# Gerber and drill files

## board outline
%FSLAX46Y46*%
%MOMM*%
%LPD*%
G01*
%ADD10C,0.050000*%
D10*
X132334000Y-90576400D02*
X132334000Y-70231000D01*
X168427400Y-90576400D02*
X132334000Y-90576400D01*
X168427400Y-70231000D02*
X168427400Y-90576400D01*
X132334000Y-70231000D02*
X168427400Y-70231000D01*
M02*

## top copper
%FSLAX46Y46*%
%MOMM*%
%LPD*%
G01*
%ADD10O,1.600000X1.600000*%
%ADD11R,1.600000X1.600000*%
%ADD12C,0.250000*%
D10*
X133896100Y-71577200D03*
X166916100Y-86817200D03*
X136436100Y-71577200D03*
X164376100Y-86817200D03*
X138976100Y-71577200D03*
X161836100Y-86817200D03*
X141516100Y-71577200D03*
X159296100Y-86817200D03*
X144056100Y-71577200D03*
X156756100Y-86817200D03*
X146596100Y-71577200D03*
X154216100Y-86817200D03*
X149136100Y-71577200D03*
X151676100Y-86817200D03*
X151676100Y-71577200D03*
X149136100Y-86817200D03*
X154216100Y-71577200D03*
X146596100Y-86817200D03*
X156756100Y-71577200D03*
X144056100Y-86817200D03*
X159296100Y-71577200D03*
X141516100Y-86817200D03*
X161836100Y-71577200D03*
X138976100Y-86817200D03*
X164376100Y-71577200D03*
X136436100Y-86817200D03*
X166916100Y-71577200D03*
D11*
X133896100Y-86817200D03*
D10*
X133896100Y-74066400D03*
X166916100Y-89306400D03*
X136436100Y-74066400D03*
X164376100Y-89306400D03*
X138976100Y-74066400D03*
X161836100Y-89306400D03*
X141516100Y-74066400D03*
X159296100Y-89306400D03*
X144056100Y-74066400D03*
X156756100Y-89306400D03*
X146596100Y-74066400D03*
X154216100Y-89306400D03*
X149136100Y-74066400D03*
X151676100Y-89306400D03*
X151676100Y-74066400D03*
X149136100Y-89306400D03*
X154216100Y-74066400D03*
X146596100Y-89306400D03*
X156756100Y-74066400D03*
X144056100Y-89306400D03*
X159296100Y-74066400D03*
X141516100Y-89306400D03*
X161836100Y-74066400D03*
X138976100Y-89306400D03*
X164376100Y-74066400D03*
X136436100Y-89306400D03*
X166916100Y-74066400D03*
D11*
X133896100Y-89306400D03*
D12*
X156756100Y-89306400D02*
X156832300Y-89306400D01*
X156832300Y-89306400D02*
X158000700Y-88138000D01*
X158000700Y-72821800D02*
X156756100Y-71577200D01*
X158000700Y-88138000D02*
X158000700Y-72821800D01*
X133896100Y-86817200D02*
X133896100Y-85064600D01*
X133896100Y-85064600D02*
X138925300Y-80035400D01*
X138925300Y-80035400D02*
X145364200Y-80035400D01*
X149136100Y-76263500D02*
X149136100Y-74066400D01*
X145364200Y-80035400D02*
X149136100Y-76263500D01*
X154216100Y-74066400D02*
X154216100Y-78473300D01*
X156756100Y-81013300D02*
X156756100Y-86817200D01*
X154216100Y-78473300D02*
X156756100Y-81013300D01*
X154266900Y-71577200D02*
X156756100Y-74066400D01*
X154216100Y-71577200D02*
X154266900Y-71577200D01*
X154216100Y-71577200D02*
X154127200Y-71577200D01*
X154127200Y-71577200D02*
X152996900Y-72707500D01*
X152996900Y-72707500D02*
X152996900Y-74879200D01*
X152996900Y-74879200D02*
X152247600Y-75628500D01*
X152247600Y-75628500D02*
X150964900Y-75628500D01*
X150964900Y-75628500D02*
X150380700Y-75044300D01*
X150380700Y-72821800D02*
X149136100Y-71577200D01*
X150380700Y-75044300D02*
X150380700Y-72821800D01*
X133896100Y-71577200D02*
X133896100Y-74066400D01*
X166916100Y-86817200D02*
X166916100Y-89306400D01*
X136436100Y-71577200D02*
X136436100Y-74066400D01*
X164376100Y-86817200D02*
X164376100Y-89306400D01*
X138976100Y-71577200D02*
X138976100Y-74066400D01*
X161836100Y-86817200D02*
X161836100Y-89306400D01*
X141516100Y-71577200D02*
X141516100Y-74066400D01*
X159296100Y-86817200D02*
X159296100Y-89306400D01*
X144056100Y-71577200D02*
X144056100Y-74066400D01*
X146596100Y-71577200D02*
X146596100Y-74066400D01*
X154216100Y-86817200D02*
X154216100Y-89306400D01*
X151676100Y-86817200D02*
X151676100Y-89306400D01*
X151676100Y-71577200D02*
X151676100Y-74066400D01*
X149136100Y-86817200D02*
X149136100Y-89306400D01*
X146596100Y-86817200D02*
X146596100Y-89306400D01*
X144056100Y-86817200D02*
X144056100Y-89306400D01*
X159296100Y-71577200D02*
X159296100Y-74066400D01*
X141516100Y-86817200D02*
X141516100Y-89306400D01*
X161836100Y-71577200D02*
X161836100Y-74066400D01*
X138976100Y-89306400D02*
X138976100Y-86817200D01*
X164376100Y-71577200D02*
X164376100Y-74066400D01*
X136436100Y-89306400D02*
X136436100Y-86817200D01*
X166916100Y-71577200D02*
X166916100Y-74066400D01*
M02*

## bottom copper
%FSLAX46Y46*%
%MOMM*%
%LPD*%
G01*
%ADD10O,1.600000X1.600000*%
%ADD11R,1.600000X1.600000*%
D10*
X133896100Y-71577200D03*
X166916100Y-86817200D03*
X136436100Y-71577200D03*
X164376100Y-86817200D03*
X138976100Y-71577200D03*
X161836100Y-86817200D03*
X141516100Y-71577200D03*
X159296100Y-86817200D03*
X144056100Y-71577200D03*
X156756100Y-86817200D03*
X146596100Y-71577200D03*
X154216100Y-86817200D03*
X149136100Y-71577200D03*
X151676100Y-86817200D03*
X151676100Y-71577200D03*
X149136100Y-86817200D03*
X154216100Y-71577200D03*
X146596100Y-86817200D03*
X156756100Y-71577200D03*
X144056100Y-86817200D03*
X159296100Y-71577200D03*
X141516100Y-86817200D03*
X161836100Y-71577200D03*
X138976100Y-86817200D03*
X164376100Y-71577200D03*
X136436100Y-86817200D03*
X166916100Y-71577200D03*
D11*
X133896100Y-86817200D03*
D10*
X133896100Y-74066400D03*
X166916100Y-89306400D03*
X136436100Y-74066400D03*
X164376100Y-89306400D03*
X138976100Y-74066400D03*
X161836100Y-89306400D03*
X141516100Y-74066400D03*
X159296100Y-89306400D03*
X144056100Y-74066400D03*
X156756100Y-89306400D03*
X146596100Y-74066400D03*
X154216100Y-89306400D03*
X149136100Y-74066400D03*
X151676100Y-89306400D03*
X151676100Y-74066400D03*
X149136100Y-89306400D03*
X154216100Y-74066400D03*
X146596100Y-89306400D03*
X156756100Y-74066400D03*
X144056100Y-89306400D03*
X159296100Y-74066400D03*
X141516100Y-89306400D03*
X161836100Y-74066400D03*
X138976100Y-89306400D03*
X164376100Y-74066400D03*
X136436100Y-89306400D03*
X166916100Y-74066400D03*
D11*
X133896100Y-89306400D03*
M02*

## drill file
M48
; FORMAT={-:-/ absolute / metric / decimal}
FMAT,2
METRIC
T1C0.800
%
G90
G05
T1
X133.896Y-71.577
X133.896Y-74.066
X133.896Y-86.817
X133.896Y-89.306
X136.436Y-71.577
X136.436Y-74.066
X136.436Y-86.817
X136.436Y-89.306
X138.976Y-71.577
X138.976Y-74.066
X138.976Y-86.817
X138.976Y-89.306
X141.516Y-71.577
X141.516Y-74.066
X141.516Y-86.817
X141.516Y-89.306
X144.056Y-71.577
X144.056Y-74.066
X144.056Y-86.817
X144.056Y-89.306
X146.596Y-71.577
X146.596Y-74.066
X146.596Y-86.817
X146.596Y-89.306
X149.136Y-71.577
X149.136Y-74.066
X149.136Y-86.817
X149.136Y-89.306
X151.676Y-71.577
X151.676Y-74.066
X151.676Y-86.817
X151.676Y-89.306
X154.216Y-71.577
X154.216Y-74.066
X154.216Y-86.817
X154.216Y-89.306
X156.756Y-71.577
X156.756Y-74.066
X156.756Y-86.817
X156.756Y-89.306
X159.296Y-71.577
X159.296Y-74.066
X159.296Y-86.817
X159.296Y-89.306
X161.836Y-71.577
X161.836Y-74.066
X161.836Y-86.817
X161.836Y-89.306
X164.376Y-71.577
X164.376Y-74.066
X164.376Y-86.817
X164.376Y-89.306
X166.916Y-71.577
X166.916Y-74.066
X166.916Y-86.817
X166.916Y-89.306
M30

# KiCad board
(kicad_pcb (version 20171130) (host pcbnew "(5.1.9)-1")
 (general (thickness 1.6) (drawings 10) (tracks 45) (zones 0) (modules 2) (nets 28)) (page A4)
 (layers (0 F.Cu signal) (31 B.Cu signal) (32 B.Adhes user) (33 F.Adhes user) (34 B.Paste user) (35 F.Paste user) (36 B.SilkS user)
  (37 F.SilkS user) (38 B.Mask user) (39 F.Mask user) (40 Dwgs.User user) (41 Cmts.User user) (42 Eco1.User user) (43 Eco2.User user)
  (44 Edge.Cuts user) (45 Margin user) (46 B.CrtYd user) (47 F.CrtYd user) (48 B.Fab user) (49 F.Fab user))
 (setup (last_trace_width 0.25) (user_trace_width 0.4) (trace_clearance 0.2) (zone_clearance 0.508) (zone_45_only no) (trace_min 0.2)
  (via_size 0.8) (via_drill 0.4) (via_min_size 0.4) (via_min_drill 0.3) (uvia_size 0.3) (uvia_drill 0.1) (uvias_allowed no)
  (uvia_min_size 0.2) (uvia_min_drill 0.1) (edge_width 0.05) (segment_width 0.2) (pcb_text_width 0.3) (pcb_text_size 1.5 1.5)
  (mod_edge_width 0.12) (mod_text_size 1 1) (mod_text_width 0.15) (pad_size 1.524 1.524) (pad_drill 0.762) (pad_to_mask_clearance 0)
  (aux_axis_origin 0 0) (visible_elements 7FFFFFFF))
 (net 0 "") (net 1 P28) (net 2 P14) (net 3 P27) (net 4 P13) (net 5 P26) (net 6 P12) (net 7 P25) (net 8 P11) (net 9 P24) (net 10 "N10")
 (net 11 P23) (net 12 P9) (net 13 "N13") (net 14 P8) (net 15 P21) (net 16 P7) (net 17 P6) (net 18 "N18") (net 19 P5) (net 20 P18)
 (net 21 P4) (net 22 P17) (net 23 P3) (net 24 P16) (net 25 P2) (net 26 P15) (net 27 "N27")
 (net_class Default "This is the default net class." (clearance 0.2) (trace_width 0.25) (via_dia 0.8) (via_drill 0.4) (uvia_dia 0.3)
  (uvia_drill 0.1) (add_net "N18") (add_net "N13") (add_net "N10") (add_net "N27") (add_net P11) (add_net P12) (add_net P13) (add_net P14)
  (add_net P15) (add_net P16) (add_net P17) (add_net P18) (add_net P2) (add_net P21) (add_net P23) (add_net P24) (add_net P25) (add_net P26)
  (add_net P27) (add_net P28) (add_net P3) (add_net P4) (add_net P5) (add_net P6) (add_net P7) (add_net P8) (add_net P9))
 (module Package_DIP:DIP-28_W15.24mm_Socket (layer F.Cu) (at 133.8961 86.8172 90)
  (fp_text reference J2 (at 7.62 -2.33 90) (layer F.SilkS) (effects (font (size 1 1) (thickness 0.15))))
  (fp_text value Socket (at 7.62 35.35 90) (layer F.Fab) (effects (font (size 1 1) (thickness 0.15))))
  (pad 28 thru_hole oval (at 15.24 0 90) (size 1.6 1.6) (drill 0.8) (layers *.Cu *.Mask) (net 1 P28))
  (pad 14 thru_hole oval (at 0 33.02 90) (size 1.6 1.6) (drill 0.8) (layers *.Cu *.Mask) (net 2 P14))
  (pad 27 thru_hole oval (at 15.24 2.54 90) (size 1.6 1.6) (drill 0.8) (layers *.Cu *.Mask) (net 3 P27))
  (pad 13 thru_hole oval (at 0 30.48 90) (size 1.6 1.6) (drill 0.8) (layers *.Cu *.Mask) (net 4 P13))
  (pad 26 thru_hole oval (at 15.24 5.08 90) (size 1.6 1.6) (drill 0.8) (layers *.Cu *.Mask) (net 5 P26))
  (pad 12 thru_hole oval (at 0 27.94 90) (size 1.6 1.6) (drill 0.8) (layers *.Cu *.Mask) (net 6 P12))
  (pad 25 thru_hole oval (at 15.24 7.62 90) (size 1.6 1.6) (drill 0.8) (layers *.Cu *.Mask) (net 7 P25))
  (pad 11 thru_hole oval (at 0 25.4 90) (size 1.6 1.6) (drill 0.8) (layers *.Cu *.Mask) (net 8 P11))
  (pad 24 thru_hole oval (at 15.24 10.16 90) (size 1.6 1.6) (drill 0.8) (layers *.Cu *.Mask) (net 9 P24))
  (pad 10 thru_hole oval (at 0 22.86 90) (size 1.6 1.6) (drill 0.8) (layers *.Cu *.Mask) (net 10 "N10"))
  (pad 23 thru_hole oval (at 15.24 12.7 90) (size 1.6 1.6) (drill 0.8) (layers *.Cu *.Mask) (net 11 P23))
  (pad 9 thru_hole oval (at 0 20.32 90) (size 1.6 1.6) (drill 0.8) (layers *.Cu *.Mask) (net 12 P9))
  (pad 22 thru_hole oval (at 15.24 15.24 90) (size 1.6 1.6) (drill 0.8) (layers *.Cu *.Mask) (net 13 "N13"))
  (pad 8 thru_hole oval (at 0 17.78 90) (size 1.6 1.6) (drill 0.8) (layers *.Cu *.Mask) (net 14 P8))
  (pad 21 thru_hole oval (at 15.24 17.78 90) (size 1.6 1.6) (drill 0.8) (layers *.Cu *.Mask) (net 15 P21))
  (pad 7 thru_hole oval (at 0 15.24 90) (size 1.6 1.6) (drill 0.8) (layers *.Cu *.Mask) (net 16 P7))
  (pad 20 thru_hole oval (at 15.24 20.32 90) (size 1.6 1.6) (drill 0.8) (layers *.Cu *.Mask) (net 13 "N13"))
  (pad 6 thru_hole oval (at 0 12.7 90) (size 1.6 1.6) (drill 0.8) (layers *.Cu *.Mask) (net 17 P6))
  (pad 19 thru_hole oval (at 15.24 22.86 90) (size 1.6 1.6) (drill 0.8) (layers *.Cu *.Mask) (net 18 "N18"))
  (pad 5 thru_hole oval (at 0 10.16 90) (size 1.6 1.6) (drill 0.8) (layers *.Cu *.Mask) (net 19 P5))
  (pad 18 thru_hole oval (at 15.24 25.4 90) (size 1.6 1.6) (drill 0.8) (layers *.Cu *.Mask) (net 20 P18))
  (pad 4 thru_hole oval (at 0 7.62 90) (size 1.6 1.6) (drill 0.8) (layers *.Cu *.Mask) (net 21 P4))
  (pad 17 thru_hole oval (at 15.24 27.94 90) (size 1.6 1.6) (drill 0.8) (layers *.Cu *.Mask) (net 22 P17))
  (pad 3 thru_hole oval (at 0 5.08 90) (size 1.6 1.6) (drill 0.8) (layers *.Cu *.Mask) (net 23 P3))
  (pad 16 thru_hole oval (at 15.24 30.48 90) (size 1.6 1.6) (drill 0.8) (layers *.Cu *.Mask) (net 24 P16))
  (pad 2 thru_hole oval (at 0 2.54 90) (size 1.6 1.6) (drill 0.8) (layers *.Cu *.Mask) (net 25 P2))
  (pad 15 thru_hole oval (at 15.24 33.02 90) (size 1.6 1.6) (drill 0.8) (layers *.Cu *.Mask) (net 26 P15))
  (pad 1 thru_hole rect (at 0 0 90) (size 1.6 1.6) (drill 0.8) (layers *.Cu *.Mask) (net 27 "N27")))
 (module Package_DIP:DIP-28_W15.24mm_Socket (layer F.Cu) (at 133.8961 89.3064 90)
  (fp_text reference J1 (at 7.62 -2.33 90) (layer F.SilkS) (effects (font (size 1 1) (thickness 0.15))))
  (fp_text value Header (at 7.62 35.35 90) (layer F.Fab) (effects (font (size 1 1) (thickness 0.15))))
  (pad 28 thru_hole oval (at 15.24 0 90) (size 1.6 1.6) (drill 0.8) (layers *.Cu *.Mask) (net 1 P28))
  (pad 14 thru_hole oval (at 0 33.02 90) (size 1.6 1.6) (drill 0.8) (layers *.Cu *.Mask) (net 2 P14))
  (pad 27 thru_hole oval (at 15.24 2.54 90) (size 1.6 1.6) (drill 0.8) (layers *.Cu *.Mask) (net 3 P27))
  (pad 13 thru_hole oval (at 0 30.48 90) (size 1.6 1.6) (drill 0.8) (layers *.Cu *.Mask) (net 4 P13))
  (pad 26 thru_hole oval (at 15.24 5.08 90) (size 1.6 1.6) (drill 0.8) (layers *.Cu *.Mask) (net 5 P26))
  (pad 12 thru_hole oval (at 0 27.94 90) (size 1.6 1.6) (drill 0.8) (layers *.Cu *.Mask) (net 6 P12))
  (pad 25 thru_hole oval (at 15.24 7.62 90) (size 1.6 1.6) (drill 0.8) (layers *.Cu *.Mask) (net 7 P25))
  (pad 11 thru_hole oval (at 0 25.4 90) (size 1.6 1.6) (drill 0.8) (layers *.Cu *.Mask) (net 8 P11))
  (pad 24 thru_hole oval (at 15.24 10.16 90) (size 1.6 1.6) (drill 0.8) (layers *.Cu *.Mask) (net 9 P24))
  (pad 10 thru_hole oval (at 0 22.86 90) (size 1.6 1.6) (drill 0.8) (layers *.Cu *.Mask) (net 18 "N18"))
  (pad 23 thru_hole oval (at 15.24 12.7 90) (size 1.6 1.6) (drill 0.8) (layers *.Cu *.Mask) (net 11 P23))
  (pad 9 thru_hole oval (at 0 20.32 90) (size 1.6 1.6) (drill 0.8) (layers *.Cu *.Mask) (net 12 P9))
  (pad 22 thru_hole oval (at 15.24 15.24 90) (size 1.6 1.6) (drill 0.8) (layers *.Cu *.Mask) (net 27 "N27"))
  (pad 8 thru_hole oval (at 0 17.78 90) (size 1.6 1.6) (drill 0.8) (layers *.Cu *.Mask) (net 14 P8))
  (pad 21 thru_hole oval (at 15.24 17.78 90) (size 1.6 1.6) (drill 0.8) (layers *.Cu *.Mask) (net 15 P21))
  (pad 7 thru_hole oval (at 0 15.24 90) (size 1.6 1.6) (drill 0.8) (layers *.Cu *.Mask) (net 16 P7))
  (pad 20 thru_hole oval (at 15.24 20.32 90) (size 1.6 1.6) (drill 0.8) (layers *.Cu *.Mask) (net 10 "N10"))
  (pad 6 thru_hole oval (at 0 12.7 90) (size 1.6 1.6) (drill 0.8) (layers *.Cu *.Mask) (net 17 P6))
  (pad 19 thru_hole oval (at 15.24 22.86 90) (size 1.6 1.6) (drill 0.8) (layers *.Cu *.Mask) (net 13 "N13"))
  (pad 5 thru_hole oval (at 0 10.16 90) (size 1.6 1.6) (drill 0.8) (layers *.Cu *.Mask) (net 19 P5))
  (pad 18 thru_hole oval (at 15.24 25.4 90) (size 1.6 1.6) (drill 0.8) (layers *.Cu *.Mask) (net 20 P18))
  (pad 4 thru_hole oval (at 0 7.62 90) (size 1.6 1.6) (drill 0.8) (layers *.Cu *.Mask) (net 21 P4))
  (pad 17 thru_hole oval (at 15.24 27.94 90) (size 1.6 1.6) (drill 0.8) (layers *.Cu *.Mask) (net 22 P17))
  (pad 3 thru_hole oval (at 0 5.08 90) (size 1.6 1.6) (drill 0.8) (layers *.Cu *.Mask) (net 23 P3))
  (pad 16 thru_hole oval (at 15.24 30.48 90) (size 1.6 1.6) (drill 0.8) (layers *.Cu *.Mask) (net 24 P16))
  (pad 2 thru_hole oval (at 0 2.54 90) (size 1.6 1.6) (drill 0.8) (layers *.Cu *.Mask) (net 25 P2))
  (pad 15 thru_hole oval (at 15.24 33.02 90) (size 1.6 1.6) (drill 0.8) (layers *.Cu *.Mask) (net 26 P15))
  (pad 1 thru_hole rect (at 0 0 90) (size 1.6 1.6) (drill 0.8) (layers *.Cu *.Mask)))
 (gr_line (start 132.334 90.5764) (end 132.334 70.231) (layer Edge.Cuts) (width 0.05))
 (gr_line (start 168.4274 90.5764) (end 132.334 90.5764) (layer Edge.Cuts) (width 0.05))
 (gr_line (start 168.4274 70.231) (end 168.4274 90.5764) (layer Edge.Cuts) (width 0.05))
 (gr_line (start 132.334 70.231) (end 168.4274 70.231) (layer Edge.Cuts) (width 0.05))
 (segment (start 156.7561 89.3064) (end 156.8323 89.3064) (width 0.25) (layer F.Cu) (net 18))
 (segment (start 156.8323 89.3064) (end 158.0007 88.138) (width 0.25) (layer F.Cu) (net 18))
 (segment (start 158.0007 72.8218) (end 156.7561 71.5772) (width 0.25) (layer F.Cu) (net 18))
 (segment (start 158.0007 88.138) (end 158.0007 72.8218) (width 0.25) (layer F.Cu) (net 18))
 (segment (start 133.8961 86.8172) (end 133.8961 85.0646) (width 0.25) (layer F.Cu) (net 27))
 (segment (start 133.8961 85.0646) (end 138.9253 80.0354) (width 0.25) (layer F.Cu) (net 27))
 (segment (start 138.9253 80.0354) (end 145.3642 80.0354) (width 0.25) (layer F.Cu) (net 27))
 (segment (start 149.1361 76.2635) (end 149.1361 74.0664) (width 0.25) (layer F.Cu) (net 27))
 (segment (start 145.3642 80.0354) (end 149.1361 76.2635) (width 0.25) (layer F.Cu) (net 27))
 (segment (start 154.2161 74.0664) (end 154.2161 78.4733) (width 0.25) (layer F.Cu) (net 10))
 (segment (start 156.7561 81.0133) (end 156.7561 86.8172) (width 0.25) (layer F.Cu) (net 10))
 (segment (start 154.2161 78.4733) (end 156.7561 81.0133) (width 0.25) (layer F.Cu) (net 10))
 (segment (start 154.2669 71.5772) (end 156.7561 74.0664) (width 0.25) (layer F.Cu) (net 13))
 (segment (start 154.2161 71.5772) (end 154.2669 71.5772) (width 0.25) (layer F.Cu) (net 13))
 (segment (start 154.2161 71.5772) (end 154.1272 71.5772) (width 0.25) (layer F.Cu) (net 13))
 (segment (start 154.1272 71.5772) (end 152.9969 72.7075) (width 0.25) (layer F.Cu) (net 13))
 (segment (start 152.9969 72.7075) (end 152.9969 74.8792) (width 0.25) (layer F.Cu) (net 13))
 (segment (start 152.9969 74.8792) (end 152.2476 75.6285) (width 0.25) (layer F.Cu) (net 13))
 (segment (start 152.2476 75.6285) (end 150.9649 75.6285) (width 0.25) (layer F.Cu) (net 13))
 (segment (start 150.9649 75.6285) (end 150.3807 75.0443) (width 0.25) (layer F.Cu) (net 13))
 (segment (start 150.3807 72.8218) (end 149.1361 71.5772) (width 0.25) (layer F.Cu) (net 13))
 (segment (start 150.3807 75.0443) (end 150.3807 72.8218) (width 0.25) (layer F.Cu) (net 13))
 (segment (start 133.8961 71.5772) (end 133.8961 74.0664) (width 0.25) (layer F.Cu) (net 1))
 (segment (start 166.9161 86.8172) (end 166.9161 89.3064) (width 0.25) (layer F.Cu) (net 2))
 (segment (start 136.4361 71.5772) (end 136.4361 74.0664) (width 0.25) (layer F.Cu) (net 3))
 (segment (start 164.3761 86.8172) (end 164.3761 89.3064) (width 0.25) (layer F.Cu) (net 4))
 (segment (start 138.9761 71.5772) (end 138.9761 74.0664) (width 0.25) (layer F.Cu) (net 5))
 (segment (start 161.8361 86.8172) (end 161.8361 89.3064) (width 0.25) (layer F.Cu) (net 6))
 (segment (start 141.5161 71.5772) (end 141.5161 74.0664) (width 0.25) (layer F.Cu) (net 7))
 (segment (start 159.2961 86.8172) (end 159.2961 89.3064) (width 0.25) (layer F.Cu) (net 8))
 (segment (start 144.0561 71.5772) (end 144.0561 74.0664) (width 0.25) (layer F.Cu) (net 9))
 (segment (start 146.5961 71.5772) (end 146.5961 74.0664) (width 0.25) (layer F.Cu) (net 11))
 (segment (start 154.2161 86.8172) (end 154.2161 89.3064) (width 0.25) (layer F.Cu) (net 12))
 (segment (start 151.6761 86.8172) (end 151.6761 89.3064) (width 0.25) (layer F.Cu) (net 14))
 (segment (start 151.6761 71.5772) (end 151.6761 74.0664) (width 0.25) (layer F.Cu) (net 15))
 (segment (start 149.1361 86.8172) (end 149.1361 89.3064) (width 0.25) (layer F.Cu) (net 16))
 (segment (start 146.5961 86.8172) (end 146.5961 89.3064) (width 0.25) (layer F.Cu) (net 17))
 (segment (start 144.0561 86.8172) (end 144.0561 89.3064) (width 0.25) (layer F.Cu) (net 19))
 (segment (start 159.2961 71.5772) (end 159.2961 74.0664) (width 0.25) (layer F.Cu) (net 20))
 (segment (start 141.5161 86.8172) (end 141.5161 89.3064) (width 0.25) (layer F.Cu) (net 21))
 (segment (start 161.8361 71.5772) (end 161.8361 74.0664) (width 0.25) (layer F.Cu) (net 22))
 (segment (start 138.9761 89.3064) (end 138.9761 86.8172) (width 0.25) (layer F.Cu) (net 23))
 (segment (start 164.3761 71.5772) (end 164.3761 74.0664) (width 0.25) (layer F.Cu) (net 24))
 (segment (start 136.4361 89.3064) (end 136.4361 86.8172) (width 0.25) (layer F.Cu) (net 25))
 (segment (start 166.9161 71.5772) (end 166.9161 74.0664) (width 0.25) (layer F.Cu) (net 26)))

